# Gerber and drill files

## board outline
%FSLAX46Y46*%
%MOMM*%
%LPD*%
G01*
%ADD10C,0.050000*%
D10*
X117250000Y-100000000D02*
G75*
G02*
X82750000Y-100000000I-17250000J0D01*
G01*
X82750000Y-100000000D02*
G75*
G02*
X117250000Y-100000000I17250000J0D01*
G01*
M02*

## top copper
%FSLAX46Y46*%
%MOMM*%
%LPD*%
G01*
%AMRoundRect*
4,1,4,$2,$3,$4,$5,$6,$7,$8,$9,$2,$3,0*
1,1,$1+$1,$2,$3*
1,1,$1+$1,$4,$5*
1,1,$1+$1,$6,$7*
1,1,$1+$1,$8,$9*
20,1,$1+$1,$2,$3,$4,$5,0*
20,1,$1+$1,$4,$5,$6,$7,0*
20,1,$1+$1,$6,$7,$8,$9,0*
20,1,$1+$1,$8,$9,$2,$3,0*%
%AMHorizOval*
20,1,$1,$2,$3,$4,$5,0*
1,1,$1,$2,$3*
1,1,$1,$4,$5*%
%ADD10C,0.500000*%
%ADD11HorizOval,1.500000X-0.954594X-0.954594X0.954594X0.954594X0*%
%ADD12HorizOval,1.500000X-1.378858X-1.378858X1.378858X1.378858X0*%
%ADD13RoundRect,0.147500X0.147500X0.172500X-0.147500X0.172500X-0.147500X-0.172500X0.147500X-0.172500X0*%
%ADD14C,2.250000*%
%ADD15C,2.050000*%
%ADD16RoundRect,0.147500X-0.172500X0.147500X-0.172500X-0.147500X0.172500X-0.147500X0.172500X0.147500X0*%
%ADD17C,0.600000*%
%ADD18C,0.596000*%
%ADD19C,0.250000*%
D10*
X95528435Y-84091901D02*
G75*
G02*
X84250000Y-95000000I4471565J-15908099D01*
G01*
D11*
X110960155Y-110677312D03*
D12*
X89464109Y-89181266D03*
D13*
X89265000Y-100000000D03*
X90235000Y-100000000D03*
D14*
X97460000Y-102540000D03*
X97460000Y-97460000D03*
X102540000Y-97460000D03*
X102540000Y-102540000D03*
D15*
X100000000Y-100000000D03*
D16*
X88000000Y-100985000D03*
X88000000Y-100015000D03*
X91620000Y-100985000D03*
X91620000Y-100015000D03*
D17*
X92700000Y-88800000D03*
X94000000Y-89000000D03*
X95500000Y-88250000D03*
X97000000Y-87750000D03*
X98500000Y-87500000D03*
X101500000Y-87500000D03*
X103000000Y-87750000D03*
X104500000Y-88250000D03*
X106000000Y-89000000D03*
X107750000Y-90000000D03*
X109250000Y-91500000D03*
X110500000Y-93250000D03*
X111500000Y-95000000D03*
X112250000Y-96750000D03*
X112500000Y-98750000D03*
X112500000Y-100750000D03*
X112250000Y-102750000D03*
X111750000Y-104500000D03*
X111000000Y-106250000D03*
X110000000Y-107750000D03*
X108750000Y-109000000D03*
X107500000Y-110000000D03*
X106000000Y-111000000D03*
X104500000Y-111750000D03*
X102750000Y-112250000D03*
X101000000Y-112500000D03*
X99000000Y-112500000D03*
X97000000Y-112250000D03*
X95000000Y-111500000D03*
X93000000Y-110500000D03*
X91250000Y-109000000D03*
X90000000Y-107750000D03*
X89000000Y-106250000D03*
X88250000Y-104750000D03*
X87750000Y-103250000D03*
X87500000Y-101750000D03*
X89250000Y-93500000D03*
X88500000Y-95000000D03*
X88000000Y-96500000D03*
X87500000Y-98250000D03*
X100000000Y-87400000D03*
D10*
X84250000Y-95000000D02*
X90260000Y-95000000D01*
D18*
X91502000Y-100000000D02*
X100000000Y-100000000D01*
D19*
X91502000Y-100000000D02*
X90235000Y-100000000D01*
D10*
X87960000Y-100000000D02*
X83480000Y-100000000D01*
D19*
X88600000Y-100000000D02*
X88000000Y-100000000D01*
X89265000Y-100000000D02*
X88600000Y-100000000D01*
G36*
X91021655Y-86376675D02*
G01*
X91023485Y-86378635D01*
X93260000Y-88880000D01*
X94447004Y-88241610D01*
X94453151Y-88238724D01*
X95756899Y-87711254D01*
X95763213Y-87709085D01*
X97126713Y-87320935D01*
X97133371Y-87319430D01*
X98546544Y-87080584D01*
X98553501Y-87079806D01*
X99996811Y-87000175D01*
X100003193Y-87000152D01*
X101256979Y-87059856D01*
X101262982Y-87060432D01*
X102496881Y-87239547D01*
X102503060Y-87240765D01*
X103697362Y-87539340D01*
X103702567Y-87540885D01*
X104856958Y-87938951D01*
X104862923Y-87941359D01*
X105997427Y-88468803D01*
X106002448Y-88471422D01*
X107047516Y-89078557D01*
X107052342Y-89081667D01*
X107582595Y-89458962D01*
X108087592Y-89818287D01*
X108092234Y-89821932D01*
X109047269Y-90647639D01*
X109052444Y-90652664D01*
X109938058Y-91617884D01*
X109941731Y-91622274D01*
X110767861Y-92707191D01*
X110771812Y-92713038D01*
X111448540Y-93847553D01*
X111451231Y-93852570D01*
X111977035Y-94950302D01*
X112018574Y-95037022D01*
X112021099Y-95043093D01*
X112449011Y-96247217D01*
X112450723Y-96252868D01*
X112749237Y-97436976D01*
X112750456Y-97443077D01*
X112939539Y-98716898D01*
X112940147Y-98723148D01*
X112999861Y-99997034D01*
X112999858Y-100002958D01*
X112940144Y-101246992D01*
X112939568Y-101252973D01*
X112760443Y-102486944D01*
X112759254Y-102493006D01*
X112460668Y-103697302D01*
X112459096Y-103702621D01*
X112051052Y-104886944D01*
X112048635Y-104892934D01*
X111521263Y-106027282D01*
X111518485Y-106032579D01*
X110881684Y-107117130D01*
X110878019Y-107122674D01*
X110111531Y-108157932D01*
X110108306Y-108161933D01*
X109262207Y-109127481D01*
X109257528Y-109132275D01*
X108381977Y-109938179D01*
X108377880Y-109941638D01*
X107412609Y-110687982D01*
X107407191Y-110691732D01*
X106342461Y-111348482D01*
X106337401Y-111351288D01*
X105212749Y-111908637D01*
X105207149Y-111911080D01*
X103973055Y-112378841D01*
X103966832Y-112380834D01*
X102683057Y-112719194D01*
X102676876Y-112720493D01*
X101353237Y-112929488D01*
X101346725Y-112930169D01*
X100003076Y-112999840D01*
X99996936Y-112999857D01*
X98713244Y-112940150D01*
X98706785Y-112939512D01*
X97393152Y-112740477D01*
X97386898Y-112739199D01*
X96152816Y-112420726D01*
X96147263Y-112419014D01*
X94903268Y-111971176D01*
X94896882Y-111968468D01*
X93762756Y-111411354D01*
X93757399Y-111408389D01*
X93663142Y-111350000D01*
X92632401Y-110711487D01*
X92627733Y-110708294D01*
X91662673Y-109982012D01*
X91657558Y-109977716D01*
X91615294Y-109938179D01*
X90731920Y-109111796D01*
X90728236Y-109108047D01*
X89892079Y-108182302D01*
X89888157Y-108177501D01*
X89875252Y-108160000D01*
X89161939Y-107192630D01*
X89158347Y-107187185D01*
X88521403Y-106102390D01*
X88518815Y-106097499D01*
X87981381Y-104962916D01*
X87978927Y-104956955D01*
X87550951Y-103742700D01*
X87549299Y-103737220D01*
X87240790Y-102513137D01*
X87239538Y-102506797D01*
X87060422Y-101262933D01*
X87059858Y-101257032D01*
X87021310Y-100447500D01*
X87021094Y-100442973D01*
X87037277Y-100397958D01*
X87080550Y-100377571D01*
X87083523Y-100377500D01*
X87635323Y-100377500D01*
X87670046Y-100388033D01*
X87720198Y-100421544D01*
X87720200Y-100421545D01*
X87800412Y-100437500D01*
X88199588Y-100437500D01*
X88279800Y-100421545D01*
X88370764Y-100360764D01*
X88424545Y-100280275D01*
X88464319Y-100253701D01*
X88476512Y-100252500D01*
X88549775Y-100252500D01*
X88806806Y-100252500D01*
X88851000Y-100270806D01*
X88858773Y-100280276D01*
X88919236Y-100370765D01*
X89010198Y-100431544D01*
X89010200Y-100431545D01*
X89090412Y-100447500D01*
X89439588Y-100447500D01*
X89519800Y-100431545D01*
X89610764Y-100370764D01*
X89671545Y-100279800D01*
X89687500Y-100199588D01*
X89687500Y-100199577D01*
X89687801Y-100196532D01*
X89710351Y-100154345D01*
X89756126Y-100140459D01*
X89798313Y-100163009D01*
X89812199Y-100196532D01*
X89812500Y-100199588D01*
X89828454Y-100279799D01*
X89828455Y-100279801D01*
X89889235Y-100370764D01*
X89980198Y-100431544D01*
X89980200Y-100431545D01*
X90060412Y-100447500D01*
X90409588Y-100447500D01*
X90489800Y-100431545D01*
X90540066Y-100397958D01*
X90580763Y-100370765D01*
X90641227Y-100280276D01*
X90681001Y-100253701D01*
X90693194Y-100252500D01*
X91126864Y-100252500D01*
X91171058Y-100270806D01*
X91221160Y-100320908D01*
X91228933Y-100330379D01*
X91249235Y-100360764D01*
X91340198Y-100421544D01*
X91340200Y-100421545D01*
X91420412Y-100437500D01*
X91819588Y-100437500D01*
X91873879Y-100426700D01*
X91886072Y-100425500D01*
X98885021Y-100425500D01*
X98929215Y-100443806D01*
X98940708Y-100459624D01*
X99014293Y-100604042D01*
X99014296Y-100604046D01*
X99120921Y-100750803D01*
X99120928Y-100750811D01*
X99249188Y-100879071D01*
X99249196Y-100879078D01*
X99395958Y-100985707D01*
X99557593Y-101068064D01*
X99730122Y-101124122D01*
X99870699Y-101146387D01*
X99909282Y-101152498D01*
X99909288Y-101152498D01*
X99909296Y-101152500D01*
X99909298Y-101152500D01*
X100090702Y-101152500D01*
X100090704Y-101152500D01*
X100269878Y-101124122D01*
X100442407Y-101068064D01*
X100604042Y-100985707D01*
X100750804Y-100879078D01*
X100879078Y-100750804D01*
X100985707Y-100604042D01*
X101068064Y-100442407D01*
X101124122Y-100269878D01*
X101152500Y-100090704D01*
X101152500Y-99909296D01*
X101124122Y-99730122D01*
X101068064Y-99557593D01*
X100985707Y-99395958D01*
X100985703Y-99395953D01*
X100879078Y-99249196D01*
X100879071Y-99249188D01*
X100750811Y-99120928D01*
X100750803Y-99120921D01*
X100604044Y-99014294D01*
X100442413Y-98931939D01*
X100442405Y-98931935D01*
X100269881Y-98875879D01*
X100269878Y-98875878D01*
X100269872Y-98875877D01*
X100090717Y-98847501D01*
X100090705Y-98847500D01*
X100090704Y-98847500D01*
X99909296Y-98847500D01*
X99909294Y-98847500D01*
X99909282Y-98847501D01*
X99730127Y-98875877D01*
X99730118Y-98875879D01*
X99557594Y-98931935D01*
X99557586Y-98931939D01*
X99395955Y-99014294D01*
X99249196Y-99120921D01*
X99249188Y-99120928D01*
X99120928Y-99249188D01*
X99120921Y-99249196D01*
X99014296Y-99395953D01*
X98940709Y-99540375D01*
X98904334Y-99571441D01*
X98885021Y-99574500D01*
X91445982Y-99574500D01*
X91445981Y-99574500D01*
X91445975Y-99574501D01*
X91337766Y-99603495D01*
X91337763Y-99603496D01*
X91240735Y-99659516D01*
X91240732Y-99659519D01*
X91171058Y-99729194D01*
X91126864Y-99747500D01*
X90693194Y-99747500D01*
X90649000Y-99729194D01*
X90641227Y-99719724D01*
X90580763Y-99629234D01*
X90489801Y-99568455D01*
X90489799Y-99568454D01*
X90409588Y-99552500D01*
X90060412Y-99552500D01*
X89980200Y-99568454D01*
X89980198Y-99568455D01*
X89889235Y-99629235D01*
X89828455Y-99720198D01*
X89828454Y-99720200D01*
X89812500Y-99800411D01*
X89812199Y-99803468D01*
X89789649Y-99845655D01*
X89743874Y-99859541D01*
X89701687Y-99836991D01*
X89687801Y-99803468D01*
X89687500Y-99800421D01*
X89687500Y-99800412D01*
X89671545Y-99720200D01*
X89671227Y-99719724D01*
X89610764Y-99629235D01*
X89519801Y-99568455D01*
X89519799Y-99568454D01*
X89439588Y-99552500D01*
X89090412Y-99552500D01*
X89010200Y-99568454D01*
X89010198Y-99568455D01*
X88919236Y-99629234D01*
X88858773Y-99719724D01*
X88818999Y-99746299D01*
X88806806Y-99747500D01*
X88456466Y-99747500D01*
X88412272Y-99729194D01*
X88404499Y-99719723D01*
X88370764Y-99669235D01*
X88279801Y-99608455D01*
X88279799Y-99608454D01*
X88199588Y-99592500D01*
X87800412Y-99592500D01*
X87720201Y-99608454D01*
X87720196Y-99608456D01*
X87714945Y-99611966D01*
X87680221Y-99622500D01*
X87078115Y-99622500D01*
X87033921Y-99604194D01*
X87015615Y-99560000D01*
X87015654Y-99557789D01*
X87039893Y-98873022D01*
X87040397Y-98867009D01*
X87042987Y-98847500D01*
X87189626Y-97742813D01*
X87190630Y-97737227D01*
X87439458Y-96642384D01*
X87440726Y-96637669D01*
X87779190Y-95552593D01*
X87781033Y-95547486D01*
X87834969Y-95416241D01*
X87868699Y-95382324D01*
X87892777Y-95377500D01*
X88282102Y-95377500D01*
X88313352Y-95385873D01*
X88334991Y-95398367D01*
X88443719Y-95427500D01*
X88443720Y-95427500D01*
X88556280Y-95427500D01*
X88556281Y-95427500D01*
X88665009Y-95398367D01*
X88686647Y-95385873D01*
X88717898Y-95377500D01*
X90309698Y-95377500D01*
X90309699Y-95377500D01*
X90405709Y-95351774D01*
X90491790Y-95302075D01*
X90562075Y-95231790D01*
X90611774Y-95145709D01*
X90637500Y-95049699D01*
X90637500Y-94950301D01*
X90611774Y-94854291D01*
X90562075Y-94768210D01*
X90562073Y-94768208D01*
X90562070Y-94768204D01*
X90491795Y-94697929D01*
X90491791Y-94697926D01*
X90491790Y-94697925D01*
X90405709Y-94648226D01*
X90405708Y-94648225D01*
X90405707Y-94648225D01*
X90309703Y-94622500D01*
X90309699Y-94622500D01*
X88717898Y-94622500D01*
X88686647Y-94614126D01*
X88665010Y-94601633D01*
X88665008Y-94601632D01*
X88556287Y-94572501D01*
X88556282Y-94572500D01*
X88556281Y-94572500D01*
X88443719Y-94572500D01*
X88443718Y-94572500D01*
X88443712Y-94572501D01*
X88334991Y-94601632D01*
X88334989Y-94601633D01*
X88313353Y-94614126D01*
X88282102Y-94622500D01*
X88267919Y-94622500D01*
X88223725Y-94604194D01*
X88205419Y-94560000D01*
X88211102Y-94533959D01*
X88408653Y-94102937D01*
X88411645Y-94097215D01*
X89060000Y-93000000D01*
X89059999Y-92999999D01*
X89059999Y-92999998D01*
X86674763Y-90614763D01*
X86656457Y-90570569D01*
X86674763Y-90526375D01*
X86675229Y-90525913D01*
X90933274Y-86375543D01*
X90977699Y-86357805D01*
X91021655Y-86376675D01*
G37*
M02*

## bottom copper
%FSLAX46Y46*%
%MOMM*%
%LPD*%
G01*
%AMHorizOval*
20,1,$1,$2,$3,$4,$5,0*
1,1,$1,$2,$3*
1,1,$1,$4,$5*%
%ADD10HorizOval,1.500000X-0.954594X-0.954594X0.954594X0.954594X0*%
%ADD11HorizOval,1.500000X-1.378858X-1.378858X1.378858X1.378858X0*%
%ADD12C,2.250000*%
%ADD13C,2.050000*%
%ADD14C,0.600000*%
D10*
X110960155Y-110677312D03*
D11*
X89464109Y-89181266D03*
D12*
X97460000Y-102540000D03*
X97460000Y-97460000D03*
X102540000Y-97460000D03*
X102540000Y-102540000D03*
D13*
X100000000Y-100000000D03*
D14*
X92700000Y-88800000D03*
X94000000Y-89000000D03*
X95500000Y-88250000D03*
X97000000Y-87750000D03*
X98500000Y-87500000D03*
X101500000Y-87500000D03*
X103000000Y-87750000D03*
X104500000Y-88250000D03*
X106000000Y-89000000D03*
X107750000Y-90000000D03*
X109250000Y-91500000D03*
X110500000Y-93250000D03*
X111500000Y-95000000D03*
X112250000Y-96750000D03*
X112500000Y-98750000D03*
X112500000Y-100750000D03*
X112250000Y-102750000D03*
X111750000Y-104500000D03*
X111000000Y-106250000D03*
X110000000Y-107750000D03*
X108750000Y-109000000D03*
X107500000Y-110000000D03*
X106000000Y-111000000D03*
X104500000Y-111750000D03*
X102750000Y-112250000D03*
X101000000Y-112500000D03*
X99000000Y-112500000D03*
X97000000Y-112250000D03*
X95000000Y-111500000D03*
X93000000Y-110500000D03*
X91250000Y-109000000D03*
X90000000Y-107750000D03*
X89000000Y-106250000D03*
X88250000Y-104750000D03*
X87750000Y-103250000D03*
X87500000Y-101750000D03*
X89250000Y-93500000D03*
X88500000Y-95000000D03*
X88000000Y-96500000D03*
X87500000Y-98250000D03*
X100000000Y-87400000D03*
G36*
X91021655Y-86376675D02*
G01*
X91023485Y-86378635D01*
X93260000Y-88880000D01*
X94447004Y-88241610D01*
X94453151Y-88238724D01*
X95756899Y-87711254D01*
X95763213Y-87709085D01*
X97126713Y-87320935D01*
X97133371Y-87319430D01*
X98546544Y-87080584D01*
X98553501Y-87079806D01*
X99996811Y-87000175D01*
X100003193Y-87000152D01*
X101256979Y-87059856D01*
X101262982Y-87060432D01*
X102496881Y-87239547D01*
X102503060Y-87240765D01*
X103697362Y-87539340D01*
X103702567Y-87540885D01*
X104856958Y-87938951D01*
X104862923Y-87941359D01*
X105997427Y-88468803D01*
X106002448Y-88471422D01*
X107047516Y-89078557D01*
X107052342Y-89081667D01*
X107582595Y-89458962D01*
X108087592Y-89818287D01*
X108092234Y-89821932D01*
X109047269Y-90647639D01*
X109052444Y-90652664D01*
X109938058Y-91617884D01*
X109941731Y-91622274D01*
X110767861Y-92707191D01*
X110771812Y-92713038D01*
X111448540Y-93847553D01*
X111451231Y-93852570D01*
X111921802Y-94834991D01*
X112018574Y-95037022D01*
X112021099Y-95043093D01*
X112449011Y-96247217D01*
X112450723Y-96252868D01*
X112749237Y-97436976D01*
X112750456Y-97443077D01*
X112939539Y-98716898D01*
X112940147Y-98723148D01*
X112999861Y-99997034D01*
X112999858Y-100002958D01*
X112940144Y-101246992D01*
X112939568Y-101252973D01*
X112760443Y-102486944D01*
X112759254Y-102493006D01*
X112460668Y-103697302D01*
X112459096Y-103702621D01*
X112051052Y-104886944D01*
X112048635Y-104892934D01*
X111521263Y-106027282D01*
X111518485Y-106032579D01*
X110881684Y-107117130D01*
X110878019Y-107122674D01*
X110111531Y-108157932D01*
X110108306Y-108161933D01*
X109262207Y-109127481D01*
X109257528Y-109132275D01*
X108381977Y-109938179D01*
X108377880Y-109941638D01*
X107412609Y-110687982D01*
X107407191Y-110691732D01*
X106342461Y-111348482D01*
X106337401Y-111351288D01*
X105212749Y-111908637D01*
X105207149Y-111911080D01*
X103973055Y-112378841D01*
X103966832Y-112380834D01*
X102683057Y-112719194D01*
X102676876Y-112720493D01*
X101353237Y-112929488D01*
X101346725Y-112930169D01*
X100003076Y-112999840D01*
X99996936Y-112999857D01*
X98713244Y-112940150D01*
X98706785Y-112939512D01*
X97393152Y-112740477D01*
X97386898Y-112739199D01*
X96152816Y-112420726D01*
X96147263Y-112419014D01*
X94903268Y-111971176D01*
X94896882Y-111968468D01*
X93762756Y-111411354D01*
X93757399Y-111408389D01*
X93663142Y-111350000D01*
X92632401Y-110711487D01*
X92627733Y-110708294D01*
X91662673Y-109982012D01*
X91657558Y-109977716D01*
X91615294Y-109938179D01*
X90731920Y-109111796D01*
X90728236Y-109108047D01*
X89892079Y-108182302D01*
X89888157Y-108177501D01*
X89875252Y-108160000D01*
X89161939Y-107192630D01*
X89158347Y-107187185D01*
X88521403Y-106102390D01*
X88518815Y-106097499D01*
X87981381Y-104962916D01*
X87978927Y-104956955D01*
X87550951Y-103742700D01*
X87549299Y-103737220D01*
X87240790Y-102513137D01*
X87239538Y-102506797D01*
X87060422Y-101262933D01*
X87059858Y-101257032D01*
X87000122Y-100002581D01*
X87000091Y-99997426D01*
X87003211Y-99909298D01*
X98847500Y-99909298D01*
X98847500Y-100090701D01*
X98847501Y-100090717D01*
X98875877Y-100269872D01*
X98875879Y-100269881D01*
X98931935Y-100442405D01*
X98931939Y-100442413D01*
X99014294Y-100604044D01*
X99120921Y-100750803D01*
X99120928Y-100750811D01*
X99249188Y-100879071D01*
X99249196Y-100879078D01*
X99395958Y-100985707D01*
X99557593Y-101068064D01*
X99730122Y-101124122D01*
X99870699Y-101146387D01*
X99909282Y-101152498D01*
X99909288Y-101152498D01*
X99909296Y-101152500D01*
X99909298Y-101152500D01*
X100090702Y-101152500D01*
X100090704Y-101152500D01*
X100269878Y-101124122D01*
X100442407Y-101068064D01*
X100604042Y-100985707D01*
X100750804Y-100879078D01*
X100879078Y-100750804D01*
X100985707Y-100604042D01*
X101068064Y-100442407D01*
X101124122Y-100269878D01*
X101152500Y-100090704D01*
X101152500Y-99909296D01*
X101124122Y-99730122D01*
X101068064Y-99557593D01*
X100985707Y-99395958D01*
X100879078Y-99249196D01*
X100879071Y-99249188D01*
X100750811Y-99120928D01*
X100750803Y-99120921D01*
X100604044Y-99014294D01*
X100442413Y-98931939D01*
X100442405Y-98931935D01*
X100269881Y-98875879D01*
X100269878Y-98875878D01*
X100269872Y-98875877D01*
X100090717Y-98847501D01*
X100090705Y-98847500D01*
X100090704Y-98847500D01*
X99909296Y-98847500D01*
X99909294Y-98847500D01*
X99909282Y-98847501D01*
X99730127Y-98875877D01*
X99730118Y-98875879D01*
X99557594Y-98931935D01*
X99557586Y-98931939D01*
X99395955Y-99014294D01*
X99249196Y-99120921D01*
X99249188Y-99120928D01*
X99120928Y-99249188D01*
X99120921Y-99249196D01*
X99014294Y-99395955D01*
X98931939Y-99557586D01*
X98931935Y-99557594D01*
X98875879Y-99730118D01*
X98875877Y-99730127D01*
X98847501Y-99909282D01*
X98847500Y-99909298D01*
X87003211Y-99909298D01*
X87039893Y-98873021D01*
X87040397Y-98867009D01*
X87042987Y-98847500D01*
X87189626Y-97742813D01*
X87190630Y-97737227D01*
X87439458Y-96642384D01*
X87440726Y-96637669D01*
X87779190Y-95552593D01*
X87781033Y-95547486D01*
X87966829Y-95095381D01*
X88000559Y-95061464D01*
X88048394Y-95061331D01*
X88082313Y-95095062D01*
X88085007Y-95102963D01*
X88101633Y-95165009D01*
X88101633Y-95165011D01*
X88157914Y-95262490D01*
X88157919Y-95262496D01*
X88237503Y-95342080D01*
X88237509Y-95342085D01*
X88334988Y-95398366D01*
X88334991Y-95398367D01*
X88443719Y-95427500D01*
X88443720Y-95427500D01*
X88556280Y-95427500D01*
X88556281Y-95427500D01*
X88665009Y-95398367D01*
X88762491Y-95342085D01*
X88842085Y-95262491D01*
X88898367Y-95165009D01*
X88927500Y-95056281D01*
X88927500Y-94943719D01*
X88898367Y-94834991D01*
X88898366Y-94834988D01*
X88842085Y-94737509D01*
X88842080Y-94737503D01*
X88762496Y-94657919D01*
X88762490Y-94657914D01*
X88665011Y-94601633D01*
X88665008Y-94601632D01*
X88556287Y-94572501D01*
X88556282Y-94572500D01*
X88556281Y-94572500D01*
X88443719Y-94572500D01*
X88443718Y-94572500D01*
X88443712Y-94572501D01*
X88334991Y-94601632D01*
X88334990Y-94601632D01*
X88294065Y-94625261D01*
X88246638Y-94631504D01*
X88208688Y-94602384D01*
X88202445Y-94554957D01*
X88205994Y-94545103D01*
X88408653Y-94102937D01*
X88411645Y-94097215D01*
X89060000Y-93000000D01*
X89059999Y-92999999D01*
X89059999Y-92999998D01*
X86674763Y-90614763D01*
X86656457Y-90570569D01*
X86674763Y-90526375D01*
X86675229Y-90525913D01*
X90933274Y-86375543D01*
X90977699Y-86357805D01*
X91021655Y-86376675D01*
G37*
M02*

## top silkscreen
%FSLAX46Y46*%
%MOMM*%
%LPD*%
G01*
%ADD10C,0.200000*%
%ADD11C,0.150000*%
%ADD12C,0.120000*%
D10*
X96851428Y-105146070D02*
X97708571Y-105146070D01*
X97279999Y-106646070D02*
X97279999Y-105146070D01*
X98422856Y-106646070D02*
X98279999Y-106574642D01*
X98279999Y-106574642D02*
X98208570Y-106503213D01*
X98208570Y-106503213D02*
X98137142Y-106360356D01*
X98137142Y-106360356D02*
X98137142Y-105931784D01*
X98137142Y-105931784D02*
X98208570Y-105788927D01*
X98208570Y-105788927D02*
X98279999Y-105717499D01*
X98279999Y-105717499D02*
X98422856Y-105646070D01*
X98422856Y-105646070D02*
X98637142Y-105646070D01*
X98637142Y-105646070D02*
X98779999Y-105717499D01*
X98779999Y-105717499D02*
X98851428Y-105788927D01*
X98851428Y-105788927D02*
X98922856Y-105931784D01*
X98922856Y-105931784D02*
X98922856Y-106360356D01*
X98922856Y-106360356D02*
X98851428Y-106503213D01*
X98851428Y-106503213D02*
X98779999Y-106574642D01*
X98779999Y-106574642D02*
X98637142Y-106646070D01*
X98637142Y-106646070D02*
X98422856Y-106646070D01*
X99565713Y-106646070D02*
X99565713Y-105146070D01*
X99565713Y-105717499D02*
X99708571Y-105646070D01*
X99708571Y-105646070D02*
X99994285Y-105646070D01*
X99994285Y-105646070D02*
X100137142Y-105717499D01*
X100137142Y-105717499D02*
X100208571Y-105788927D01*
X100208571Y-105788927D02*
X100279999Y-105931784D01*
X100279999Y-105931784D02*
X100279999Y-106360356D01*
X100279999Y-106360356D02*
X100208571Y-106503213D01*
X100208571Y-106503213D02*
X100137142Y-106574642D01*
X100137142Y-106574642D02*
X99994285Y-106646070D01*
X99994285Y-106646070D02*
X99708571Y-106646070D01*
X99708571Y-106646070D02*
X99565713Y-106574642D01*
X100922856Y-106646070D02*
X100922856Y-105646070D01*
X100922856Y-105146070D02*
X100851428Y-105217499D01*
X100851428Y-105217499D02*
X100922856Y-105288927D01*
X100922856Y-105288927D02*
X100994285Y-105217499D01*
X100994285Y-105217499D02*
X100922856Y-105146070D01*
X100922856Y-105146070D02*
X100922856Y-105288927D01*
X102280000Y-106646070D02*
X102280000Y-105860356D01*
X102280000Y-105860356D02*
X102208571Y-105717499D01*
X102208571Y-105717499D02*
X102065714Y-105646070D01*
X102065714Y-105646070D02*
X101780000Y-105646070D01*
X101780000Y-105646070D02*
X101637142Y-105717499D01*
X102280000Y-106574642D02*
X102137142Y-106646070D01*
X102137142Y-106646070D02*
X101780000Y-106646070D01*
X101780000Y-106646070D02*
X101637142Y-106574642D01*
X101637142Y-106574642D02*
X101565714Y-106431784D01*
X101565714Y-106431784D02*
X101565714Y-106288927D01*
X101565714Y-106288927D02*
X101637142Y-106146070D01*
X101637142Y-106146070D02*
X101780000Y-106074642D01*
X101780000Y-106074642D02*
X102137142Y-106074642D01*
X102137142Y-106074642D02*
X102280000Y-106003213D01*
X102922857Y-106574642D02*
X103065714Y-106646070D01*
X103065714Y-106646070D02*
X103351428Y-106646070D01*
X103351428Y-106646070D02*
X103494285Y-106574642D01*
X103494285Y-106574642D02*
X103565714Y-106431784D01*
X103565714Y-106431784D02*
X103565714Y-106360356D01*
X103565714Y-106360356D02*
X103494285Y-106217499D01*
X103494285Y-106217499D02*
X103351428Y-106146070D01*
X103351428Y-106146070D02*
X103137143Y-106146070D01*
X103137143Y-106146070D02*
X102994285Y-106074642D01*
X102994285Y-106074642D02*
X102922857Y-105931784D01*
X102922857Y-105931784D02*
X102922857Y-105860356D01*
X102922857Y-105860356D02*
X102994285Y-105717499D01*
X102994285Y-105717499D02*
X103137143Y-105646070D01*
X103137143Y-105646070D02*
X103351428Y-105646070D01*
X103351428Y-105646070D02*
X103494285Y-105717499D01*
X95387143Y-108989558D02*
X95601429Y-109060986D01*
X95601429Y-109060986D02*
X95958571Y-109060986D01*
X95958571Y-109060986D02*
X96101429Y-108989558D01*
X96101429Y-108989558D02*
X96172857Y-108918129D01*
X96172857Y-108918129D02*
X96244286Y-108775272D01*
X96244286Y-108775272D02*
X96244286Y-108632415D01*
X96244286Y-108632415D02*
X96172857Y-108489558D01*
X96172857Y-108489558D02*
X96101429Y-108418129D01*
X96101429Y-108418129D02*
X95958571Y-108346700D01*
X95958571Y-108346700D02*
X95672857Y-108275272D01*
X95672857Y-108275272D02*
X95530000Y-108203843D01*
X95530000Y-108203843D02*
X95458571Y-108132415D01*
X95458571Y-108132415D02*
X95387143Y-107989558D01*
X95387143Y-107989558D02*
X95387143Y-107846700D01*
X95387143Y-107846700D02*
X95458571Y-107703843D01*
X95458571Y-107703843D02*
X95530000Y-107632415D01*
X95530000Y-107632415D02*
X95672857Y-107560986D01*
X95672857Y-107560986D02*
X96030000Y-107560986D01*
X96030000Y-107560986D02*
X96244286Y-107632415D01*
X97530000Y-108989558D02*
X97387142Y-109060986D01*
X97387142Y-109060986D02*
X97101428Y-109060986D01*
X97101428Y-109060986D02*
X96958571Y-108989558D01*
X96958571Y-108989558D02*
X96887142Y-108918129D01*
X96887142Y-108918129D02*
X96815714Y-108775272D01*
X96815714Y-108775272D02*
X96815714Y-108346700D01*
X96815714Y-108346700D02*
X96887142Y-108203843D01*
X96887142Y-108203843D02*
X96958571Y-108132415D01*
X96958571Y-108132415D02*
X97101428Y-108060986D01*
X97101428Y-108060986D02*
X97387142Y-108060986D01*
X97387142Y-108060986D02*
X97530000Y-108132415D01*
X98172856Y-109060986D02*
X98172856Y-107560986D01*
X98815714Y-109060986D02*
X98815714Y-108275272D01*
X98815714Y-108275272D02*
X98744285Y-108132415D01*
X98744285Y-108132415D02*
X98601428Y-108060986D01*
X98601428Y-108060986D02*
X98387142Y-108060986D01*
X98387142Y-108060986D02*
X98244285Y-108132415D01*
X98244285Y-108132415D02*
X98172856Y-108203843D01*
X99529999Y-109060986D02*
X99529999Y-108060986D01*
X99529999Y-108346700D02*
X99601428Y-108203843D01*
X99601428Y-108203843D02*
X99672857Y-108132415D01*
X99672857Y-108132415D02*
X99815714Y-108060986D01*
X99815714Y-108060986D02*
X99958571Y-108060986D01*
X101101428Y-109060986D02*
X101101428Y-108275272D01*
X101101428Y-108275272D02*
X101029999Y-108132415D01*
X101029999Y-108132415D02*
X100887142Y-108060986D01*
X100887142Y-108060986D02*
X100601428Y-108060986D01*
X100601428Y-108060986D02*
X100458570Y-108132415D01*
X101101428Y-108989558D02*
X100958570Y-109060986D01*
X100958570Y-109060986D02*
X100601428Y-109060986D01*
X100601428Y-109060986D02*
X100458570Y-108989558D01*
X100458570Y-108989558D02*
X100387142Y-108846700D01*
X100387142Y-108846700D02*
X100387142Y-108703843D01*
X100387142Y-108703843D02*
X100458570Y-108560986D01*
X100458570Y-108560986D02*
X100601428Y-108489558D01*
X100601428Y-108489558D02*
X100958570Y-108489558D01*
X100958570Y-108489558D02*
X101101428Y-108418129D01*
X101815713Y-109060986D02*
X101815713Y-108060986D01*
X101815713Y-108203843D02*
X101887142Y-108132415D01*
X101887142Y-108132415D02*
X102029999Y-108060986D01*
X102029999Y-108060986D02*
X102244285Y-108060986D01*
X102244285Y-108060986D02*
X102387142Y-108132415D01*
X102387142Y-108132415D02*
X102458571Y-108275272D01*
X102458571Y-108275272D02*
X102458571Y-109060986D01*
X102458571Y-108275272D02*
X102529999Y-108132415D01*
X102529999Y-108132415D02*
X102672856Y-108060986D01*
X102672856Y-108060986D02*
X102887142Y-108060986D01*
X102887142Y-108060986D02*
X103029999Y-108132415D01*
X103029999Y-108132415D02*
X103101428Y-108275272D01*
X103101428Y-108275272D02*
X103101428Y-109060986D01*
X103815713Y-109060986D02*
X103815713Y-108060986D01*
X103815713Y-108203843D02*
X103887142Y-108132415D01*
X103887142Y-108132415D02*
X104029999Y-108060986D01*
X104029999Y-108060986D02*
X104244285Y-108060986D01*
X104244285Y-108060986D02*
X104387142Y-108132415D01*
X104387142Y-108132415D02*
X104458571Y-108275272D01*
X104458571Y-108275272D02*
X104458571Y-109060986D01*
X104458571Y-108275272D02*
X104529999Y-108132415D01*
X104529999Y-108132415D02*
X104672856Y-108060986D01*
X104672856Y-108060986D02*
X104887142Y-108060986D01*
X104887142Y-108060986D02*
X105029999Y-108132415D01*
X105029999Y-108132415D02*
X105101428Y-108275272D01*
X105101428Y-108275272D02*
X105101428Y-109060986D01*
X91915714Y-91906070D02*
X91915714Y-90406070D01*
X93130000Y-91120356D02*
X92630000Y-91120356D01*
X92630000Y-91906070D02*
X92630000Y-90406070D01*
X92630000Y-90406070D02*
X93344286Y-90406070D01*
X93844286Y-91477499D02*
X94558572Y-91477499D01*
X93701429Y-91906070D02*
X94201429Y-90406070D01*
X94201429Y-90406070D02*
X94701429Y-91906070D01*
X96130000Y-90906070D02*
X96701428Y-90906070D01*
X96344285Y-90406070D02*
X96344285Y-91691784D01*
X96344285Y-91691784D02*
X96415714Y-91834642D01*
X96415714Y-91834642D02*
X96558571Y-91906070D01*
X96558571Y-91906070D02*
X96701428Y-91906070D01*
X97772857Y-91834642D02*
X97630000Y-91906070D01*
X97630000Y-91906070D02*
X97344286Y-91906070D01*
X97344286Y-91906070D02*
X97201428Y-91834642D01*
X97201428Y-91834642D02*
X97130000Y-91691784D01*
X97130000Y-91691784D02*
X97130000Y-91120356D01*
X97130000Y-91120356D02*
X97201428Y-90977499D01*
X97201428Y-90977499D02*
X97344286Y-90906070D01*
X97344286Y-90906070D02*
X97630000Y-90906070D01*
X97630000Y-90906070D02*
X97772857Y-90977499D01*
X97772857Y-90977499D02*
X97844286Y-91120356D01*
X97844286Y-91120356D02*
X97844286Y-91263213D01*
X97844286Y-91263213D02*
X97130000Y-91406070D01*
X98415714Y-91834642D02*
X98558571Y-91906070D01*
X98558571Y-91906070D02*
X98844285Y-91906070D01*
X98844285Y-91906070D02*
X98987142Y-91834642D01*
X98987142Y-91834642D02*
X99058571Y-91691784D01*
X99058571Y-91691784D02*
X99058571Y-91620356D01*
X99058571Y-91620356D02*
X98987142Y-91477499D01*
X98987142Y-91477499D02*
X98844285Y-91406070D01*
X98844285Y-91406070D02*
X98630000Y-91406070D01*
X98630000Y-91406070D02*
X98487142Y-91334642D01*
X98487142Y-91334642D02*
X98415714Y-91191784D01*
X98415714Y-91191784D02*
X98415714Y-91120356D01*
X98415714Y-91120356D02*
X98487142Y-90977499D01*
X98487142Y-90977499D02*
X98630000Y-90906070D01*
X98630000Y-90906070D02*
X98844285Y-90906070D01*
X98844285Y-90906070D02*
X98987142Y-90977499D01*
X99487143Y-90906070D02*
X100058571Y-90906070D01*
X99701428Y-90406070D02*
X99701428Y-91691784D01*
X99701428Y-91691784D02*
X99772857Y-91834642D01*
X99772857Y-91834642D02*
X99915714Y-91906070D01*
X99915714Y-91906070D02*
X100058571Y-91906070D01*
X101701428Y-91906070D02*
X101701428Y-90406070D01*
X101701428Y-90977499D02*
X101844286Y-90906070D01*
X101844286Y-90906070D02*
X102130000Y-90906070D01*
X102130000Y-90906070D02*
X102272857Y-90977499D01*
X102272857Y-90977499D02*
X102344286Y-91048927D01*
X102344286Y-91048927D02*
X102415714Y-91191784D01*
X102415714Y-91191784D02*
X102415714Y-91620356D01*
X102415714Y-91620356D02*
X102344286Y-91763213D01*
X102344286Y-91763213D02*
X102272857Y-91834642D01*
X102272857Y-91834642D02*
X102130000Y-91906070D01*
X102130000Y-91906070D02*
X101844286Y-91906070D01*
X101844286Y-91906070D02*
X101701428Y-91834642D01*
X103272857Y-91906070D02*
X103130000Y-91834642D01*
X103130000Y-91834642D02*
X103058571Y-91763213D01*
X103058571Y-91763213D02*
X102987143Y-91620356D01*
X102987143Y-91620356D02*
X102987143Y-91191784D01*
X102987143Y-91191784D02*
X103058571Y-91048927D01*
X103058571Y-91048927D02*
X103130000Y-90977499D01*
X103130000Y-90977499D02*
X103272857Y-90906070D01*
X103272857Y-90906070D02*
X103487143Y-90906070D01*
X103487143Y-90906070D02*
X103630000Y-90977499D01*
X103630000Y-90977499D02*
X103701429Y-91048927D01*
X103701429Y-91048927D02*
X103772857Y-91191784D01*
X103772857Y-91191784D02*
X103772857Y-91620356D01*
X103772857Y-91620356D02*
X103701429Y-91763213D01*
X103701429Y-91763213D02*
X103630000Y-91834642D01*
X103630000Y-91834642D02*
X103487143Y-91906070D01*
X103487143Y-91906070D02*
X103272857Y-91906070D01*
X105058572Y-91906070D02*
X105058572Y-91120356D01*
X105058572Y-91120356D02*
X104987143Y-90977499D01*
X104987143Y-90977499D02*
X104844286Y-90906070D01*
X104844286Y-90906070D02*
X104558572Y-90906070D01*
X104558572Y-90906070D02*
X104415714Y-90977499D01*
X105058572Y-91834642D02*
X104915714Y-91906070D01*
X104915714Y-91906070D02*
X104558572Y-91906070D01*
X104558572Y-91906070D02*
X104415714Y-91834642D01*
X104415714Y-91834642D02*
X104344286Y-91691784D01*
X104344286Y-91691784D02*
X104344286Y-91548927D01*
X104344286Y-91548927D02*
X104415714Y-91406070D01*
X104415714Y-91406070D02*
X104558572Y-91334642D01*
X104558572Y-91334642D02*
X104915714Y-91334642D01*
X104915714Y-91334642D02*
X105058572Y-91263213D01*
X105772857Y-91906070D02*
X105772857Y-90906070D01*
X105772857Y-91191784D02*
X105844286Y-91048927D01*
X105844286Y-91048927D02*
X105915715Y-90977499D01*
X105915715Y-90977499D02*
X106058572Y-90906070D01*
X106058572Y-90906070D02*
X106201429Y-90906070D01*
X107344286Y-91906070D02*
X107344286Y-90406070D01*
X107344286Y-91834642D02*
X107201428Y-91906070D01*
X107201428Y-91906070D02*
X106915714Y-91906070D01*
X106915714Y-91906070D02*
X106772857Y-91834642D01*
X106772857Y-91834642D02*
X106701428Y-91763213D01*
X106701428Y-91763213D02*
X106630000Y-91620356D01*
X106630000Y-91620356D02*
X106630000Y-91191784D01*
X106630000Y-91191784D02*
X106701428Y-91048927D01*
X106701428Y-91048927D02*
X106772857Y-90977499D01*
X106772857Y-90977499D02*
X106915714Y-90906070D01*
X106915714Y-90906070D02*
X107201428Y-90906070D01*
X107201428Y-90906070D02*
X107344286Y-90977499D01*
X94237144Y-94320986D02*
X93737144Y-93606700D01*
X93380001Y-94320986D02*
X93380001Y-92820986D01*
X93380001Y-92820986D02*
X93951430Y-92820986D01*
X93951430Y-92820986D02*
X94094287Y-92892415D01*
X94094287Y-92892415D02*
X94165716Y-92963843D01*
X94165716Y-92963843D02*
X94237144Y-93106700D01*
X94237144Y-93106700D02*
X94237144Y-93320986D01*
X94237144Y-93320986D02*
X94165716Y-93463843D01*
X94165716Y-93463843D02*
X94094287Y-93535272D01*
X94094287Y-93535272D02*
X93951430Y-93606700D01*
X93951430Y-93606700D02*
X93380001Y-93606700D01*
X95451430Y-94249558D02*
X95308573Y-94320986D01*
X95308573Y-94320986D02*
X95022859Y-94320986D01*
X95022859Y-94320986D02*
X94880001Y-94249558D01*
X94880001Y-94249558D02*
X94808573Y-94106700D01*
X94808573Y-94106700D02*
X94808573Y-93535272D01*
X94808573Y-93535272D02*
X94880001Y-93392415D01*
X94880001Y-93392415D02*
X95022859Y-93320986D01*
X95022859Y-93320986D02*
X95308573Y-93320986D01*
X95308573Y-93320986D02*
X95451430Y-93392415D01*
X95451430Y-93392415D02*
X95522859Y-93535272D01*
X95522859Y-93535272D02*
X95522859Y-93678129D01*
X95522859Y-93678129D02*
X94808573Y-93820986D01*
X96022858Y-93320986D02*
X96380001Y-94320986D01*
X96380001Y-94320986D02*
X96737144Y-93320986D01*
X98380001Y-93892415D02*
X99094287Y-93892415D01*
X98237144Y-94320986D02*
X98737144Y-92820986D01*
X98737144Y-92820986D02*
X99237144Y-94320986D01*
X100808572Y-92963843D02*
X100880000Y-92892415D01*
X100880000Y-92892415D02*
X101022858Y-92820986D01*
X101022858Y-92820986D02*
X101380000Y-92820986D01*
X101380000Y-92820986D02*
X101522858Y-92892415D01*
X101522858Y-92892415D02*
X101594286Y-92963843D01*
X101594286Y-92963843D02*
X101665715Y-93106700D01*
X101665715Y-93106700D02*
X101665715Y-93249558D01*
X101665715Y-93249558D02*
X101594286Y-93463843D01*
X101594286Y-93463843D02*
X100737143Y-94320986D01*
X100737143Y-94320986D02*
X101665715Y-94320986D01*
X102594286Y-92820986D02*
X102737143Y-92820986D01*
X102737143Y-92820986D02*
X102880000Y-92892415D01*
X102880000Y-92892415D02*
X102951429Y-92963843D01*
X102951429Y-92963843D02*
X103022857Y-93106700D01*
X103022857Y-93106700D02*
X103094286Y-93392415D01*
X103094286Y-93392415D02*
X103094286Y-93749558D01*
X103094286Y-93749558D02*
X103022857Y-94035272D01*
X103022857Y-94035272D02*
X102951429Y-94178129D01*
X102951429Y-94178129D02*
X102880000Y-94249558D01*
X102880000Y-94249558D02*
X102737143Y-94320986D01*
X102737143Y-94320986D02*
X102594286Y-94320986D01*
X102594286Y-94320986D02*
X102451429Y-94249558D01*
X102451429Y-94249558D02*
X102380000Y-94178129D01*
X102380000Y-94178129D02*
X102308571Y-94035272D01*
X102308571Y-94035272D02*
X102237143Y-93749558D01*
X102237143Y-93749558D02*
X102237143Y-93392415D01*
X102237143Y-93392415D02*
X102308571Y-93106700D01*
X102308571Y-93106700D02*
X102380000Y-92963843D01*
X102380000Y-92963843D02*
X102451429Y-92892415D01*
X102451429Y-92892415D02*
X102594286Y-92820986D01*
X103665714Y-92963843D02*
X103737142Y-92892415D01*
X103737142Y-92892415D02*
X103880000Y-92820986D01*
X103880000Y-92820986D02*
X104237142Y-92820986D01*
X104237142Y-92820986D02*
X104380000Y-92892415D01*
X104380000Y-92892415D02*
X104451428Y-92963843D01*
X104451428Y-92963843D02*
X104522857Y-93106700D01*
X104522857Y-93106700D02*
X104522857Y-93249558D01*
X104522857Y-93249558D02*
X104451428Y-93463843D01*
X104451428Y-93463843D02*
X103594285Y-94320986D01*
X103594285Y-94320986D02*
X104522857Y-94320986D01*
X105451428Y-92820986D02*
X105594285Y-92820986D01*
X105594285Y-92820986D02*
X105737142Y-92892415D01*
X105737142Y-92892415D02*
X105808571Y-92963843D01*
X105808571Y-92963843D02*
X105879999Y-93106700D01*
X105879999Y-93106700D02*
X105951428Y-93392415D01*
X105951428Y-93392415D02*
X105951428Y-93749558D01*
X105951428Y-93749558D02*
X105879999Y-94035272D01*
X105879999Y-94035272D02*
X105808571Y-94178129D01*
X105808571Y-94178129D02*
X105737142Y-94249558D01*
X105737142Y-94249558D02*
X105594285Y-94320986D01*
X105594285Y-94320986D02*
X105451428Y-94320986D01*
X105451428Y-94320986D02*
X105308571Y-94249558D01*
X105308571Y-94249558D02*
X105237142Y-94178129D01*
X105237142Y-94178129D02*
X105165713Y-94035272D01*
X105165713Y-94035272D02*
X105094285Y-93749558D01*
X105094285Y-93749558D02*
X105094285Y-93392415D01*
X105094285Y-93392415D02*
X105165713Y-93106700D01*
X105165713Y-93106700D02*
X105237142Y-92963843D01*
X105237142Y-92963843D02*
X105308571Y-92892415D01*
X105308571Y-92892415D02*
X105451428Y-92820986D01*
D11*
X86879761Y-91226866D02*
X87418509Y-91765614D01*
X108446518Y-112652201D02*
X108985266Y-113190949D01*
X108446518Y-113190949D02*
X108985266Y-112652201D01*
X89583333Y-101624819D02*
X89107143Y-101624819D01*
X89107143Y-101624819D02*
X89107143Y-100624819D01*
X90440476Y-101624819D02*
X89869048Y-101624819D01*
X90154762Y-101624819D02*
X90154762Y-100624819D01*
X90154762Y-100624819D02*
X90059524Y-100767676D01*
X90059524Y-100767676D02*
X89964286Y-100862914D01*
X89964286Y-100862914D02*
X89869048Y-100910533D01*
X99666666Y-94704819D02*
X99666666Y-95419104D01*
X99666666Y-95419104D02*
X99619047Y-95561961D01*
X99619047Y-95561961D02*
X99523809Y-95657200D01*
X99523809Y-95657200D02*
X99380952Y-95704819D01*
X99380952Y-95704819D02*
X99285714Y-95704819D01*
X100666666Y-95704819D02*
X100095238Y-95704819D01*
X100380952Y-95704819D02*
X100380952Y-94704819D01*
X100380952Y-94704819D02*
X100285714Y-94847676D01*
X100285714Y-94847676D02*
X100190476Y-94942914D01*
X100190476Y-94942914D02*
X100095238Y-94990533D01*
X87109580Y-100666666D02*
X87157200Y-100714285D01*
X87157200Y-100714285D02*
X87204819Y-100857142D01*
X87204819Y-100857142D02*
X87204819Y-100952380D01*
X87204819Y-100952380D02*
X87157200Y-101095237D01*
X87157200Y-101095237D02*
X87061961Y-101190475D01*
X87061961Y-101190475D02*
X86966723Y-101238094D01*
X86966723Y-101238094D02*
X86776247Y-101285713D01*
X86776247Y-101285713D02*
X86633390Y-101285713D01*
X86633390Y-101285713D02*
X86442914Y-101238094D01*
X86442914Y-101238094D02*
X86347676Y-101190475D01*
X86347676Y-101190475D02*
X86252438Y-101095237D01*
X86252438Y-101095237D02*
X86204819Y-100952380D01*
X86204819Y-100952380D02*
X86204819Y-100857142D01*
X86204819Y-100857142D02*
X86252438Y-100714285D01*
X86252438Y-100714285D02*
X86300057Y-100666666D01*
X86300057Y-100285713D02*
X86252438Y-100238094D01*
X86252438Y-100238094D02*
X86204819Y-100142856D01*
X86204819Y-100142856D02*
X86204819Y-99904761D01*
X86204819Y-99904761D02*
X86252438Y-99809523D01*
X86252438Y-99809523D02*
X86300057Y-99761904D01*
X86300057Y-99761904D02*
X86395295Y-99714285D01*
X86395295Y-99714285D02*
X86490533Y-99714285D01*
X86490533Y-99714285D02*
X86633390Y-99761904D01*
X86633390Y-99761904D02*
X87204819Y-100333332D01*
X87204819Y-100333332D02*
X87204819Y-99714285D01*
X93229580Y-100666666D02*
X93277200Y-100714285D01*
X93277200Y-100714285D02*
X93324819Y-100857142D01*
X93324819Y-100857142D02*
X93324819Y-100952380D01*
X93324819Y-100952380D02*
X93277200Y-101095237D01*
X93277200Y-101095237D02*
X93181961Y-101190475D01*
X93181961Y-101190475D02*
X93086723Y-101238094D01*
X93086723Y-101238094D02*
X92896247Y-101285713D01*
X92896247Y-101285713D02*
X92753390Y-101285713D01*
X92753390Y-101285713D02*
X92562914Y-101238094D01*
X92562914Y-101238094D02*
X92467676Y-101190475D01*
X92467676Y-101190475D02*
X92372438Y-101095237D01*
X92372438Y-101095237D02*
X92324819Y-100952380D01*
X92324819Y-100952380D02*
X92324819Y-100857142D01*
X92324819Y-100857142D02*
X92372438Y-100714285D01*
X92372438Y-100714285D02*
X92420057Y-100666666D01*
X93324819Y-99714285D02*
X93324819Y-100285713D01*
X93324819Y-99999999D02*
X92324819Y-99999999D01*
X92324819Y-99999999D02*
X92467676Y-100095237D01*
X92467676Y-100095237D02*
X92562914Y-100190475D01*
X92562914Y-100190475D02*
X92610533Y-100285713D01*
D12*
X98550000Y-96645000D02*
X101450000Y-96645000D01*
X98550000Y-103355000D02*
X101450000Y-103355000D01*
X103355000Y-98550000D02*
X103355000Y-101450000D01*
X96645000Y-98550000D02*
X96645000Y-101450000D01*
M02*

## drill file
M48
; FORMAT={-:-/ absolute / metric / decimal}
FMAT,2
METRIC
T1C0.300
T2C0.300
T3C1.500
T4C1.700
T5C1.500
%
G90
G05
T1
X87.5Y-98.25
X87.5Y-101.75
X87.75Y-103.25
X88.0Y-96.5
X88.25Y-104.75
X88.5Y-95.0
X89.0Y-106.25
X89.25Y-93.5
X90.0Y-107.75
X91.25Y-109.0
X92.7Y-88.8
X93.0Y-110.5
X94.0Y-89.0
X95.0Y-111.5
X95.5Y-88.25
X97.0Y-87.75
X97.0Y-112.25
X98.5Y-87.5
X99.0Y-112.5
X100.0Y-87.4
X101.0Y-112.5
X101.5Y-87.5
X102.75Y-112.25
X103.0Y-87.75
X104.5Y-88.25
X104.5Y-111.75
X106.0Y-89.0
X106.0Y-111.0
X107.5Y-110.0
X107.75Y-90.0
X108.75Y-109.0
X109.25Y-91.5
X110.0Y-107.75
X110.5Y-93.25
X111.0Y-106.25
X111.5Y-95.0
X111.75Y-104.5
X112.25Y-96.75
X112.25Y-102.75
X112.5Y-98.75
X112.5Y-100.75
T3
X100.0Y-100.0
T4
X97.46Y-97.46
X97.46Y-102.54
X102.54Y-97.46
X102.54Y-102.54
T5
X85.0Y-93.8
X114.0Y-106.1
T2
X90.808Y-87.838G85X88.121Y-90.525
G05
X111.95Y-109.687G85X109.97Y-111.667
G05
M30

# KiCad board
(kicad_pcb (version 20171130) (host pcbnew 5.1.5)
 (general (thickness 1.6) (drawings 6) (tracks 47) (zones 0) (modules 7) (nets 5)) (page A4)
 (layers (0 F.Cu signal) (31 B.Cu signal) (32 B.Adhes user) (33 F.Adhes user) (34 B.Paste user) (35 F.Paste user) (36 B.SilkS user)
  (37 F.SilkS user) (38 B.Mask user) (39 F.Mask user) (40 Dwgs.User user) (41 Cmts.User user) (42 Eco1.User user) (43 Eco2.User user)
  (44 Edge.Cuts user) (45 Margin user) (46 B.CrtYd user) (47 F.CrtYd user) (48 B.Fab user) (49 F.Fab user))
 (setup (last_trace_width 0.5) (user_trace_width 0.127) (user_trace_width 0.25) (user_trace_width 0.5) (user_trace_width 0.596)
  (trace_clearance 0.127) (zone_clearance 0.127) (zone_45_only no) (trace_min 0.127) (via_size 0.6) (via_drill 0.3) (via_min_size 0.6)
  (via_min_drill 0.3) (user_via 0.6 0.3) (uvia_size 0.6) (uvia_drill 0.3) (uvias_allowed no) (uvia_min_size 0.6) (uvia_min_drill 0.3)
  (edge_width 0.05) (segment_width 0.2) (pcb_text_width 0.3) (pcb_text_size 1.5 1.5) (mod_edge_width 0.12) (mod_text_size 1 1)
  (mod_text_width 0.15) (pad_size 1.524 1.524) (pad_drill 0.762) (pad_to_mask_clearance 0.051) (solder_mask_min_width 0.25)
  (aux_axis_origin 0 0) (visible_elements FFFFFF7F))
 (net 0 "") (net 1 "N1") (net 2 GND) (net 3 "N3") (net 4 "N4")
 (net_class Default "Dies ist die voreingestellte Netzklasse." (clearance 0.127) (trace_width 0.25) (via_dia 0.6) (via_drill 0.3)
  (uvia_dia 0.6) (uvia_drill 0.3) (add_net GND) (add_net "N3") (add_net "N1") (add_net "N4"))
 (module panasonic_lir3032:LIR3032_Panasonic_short (layer B.Cu) (at 100 100 315)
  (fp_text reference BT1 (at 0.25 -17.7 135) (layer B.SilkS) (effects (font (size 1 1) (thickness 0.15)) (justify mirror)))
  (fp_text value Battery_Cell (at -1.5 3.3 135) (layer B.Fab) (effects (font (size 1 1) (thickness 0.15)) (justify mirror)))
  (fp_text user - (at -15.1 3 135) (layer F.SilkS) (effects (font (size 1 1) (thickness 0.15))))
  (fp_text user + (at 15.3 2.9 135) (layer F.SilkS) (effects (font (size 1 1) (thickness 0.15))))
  (pad 1 thru_hole oval (at 15.3 -0.2 315) (size 1.5 4.2) (drill oval 0.3 3.1) (layers *.Cu *.Mask) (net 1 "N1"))
  (pad 2 thru_hole oval (at -15.1 -0.2 315) (size 1.5 5.4) (drill oval 0.3 4.1) (layers *.Cu *.Mask) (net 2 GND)))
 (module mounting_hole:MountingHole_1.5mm (layer F.Cu) (at 114 106.1)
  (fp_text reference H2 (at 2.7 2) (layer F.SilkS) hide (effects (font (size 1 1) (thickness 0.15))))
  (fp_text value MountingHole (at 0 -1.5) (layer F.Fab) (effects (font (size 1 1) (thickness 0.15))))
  (pad "" np_thru_hole oval (at 0 0) (size 1.5 1.5) (drill 1.5) (layers *.Cu *.Mask)))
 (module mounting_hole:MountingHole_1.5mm (layer F.Cu) (at 85 93.8)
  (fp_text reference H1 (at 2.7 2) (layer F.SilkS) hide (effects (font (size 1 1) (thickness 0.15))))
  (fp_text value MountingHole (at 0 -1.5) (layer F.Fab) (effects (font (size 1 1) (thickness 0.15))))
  (pad "" np_thru_hole oval (at 0 0) (size 1.5 1.5) (drill 1.5) (layers *.Cu *.Mask)))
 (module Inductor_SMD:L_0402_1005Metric (layer F.Cu) (at 89.75 100 180)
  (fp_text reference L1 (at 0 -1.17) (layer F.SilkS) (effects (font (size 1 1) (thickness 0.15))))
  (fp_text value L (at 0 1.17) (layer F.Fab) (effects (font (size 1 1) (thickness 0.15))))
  (pad 2 smd roundrect (at 0.485 0 180) (size 0.59 0.64) (layers F.Cu F.Paste F.Mask) (roundrect_rratio 0.25) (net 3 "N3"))
  (pad 1 smd roundrect (at -0.485 0 180) (size 0.59 0.64) (layers F.Cu F.Paste F.Mask) (roundrect_rratio 0.25) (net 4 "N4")))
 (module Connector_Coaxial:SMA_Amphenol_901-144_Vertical (layer F.Cu) (at 100 100)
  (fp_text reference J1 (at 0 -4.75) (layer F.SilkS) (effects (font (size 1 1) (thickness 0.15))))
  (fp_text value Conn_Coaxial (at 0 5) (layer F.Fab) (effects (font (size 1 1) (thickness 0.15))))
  (fp_line (start -1.45 -3.355) (end 1.45 -3.355) (layer F.SilkS) (width 0.12))
  (fp_line (start -1.45 3.355) (end 1.45 3.355) (layer F.SilkS) (width 0.12))
  (fp_line (start 3.355 -1.45) (end 3.355 1.45) (layer F.SilkS) (width 0.12))
  (fp_line (start -3.355 -1.45) (end -3.355 1.45) (layer F.SilkS) (width 0.12))
  (pad 2 thru_hole circle (at -2.54 2.54) (size 2.25 2.25) (drill 1.7) (layers *.Cu *.Mask) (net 2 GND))
  (pad 2 thru_hole circle (at -2.54 -2.54) (size 2.25 2.25) (drill 1.7) (layers *.Cu *.Mask) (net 2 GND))
  (pad 2 thru_hole circle (at 2.54 -2.54) (size 2.25 2.25) (drill 1.7) (layers *.Cu *.Mask) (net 2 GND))
  (pad 2 thru_hole circle (at 2.54 2.54) (size 2.25 2.25) (drill 1.7) (layers *.Cu *.Mask) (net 2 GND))
  (pad 1 thru_hole circle (at 0 0) (size 2.05 2.05) (drill 1.5) (layers *.Cu *.Mask) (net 4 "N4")))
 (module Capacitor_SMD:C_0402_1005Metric (layer F.Cu) (at 88 100.5 270)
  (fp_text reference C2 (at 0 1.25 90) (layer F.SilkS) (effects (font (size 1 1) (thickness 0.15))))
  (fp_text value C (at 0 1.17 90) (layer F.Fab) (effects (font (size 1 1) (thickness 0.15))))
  (pad 2 smd roundrect (at 0.485 0 270) (size 0.59 0.64) (layers F.Cu F.Paste F.Mask) (roundrect_rratio 0.25) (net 2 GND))
  (pad 1 smd roundrect (at -0.485 0 270) (size 0.59 0.64) (layers F.Cu F.Paste F.Mask) (roundrect_rratio 0.25) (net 3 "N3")))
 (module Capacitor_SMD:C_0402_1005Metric (layer F.Cu) (at 91.62 100.5 270)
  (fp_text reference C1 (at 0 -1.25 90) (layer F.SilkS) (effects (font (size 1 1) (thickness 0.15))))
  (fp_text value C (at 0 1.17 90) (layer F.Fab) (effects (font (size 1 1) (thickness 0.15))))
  (pad 2 smd roundrect (at 0.485 0 270) (size 0.59 0.64) (layers F.Cu F.Paste F.Mask) (roundrect_rratio 0.25) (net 2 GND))
  (pad 1 smd roundrect (at -0.485 0 270) (size 0.59 0.64) (layers F.Cu F.Paste F.Mask) (roundrect_rratio 0.25) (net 4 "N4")))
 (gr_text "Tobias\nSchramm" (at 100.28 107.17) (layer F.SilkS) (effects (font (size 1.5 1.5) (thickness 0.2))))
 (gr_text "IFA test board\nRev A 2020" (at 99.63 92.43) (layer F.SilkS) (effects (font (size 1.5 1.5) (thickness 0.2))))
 (gr_arc (start 100 100) (end 84.25 95) (angle -303.312578) (layer F.Cu) (width 0.5))
 (gr_circle (center 100 100) (end 117.25 100) (layer Edge.Cuts) (width 0.05))
 (segment (start 84.25 95) (end 90.26 95) (width 0.5) (layer F.Cu) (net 2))
 (via (at 92.7 88.8) (size 0.6) (drill 0.3) (layers F.Cu B.Cu) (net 2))
 (via (at 94 89) (size 0.6) (drill 0.3) (layers F.Cu B.Cu) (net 2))
 (via (at 95.5 88.25) (size 0.6) (drill 0.3) (layers F.Cu B.Cu) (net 2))
 (via (at 97 87.75) (size 0.6) (drill 0.3) (layers F.Cu B.Cu) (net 2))
 (via (at 98.5 87.5) (size 0.6) (drill 0.3) (layers F.Cu B.Cu) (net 2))
 (via (at 101.5 87.5) (size 0.6) (drill 0.3) (layers F.Cu B.Cu) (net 2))
 (via (at 103 87.75) (size 0.6) (drill 0.3) (layers F.Cu B.Cu) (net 2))
 (via (at 104.5 88.25) (size 0.6) (drill 0.3) (layers F.Cu B.Cu) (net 2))
 (via (at 106 89) (size 0.6) (drill 0.3) (layers F.Cu B.Cu) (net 2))
 (via (at 107.75 90) (size 0.6) (drill 0.3) (layers F.Cu B.Cu) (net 2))
 (via (at 109.25 91.5) (size 0.6) (drill 0.3) (layers F.Cu B.Cu) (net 2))
 (via (at 110.5 93.25) (size 0.6) (drill 0.3) (layers F.Cu B.Cu) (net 2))
 (via (at 111.5 95) (size 0.6) (drill 0.3) (layers F.Cu B.Cu) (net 2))
 (via (at 112.25 96.75) (size 0.6) (drill 0.3) (layers F.Cu B.Cu) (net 2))
 (via (at 112.5 98.75) (size 0.6) (drill 0.3) (layers F.Cu B.Cu) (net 2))
 (via (at 112.5 100.75) (size 0.6) (drill 0.3) (layers F.Cu B.Cu) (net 2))
 (via (at 112.25 102.75) (size 0.6) (drill 0.3) (layers F.Cu B.Cu) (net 2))
 (via (at 111.75 104.5) (size 0.6) (drill 0.3) (layers F.Cu B.Cu) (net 2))
 (via (at 111 106.25) (size 0.6) (drill 0.3) (layers F.Cu B.Cu) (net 2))
 (via (at 110 107.75) (size 0.6) (drill 0.3) (layers F.Cu B.Cu) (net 2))
 (via (at 108.75 109) (size 0.6) (drill 0.3) (layers F.Cu B.Cu) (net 2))
 (via (at 107.5 110) (size 0.6) (drill 0.3) (layers F.Cu B.Cu) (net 2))
 (via (at 106 111) (size 0.6) (drill 0.3) (layers F.Cu B.Cu) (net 2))
 (via (at 104.5 111.75) (size 0.6) (drill 0.3) (layers F.Cu B.Cu) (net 2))
 (via (at 102.75 112.25) (size 0.6) (drill 0.3) (layers F.Cu B.Cu) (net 2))
 (via (at 101 112.5) (size 0.6) (drill 0.3) (layers F.Cu B.Cu) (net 2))
 (via (at 99 112.5) (size 0.6) (drill 0.3) (layers F.Cu B.Cu) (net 2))
 (via (at 97 112.25) (size 0.6) (drill 0.3) (layers F.Cu B.Cu) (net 2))
 (via (at 95 111.5) (size 0.6) (drill 0.3) (layers F.Cu B.Cu) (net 2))
 (via (at 93 110.5) (size 0.6) (drill 0.3) (layers F.Cu B.Cu) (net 2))
 (via (at 91.25 109) (size 0.6) (drill 0.3) (layers F.Cu B.Cu) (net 2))
 (via (at 90 107.75) (size 0.6) (drill 0.3) (layers F.Cu B.Cu) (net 2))
 (via (at 89 106.25) (size 0.6) (drill 0.3) (layers F.Cu B.Cu) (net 2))
 (via (at 88.25 104.75) (size 0.6) (drill 0.3) (layers F.Cu B.Cu) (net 2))
 (via (at 87.75 103.25) (size 0.6) (drill 0.3) (layers F.Cu B.Cu) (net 2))
 (via (at 87.5 101.75) (size 0.6) (drill 0.3) (layers F.Cu B.Cu) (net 2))
 (via (at 89.25 93.5) (size 0.6) (drill 0.3) (layers F.Cu B.Cu) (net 2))
 (via (at 88.5 95) (size 0.6) (drill 0.3) (layers F.Cu B.Cu) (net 2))
 (via (at 88 96.5) (size 0.6) (drill 0.3) (layers F.Cu B.Cu) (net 2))
 (via (at 87.5 98.25) (size 0.6) (drill 0.3) (layers F.Cu B.Cu) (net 2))
 (via (at 100 87.4) (size 0.6) (drill 0.3) (layers F.Cu B.Cu) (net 2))
 (segment (start 91.502 100) (end 100 100) (width 0.596) (layer F.Cu) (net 4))
 (segment (start 91.502 100) (end 90.235 100) (width 0.25) (layer F.Cu) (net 4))
 (segment (start 87.96 100) (end 83.48 100) (width 0.5) (layer F.Cu) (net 3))
 (segment (start 88.6 100) (end 88 100) (width 0.25) (layer F.Cu) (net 3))
 (segment (start 89.265 100) (end 88.6 100) (width 0.25) (layer F.Cu) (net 3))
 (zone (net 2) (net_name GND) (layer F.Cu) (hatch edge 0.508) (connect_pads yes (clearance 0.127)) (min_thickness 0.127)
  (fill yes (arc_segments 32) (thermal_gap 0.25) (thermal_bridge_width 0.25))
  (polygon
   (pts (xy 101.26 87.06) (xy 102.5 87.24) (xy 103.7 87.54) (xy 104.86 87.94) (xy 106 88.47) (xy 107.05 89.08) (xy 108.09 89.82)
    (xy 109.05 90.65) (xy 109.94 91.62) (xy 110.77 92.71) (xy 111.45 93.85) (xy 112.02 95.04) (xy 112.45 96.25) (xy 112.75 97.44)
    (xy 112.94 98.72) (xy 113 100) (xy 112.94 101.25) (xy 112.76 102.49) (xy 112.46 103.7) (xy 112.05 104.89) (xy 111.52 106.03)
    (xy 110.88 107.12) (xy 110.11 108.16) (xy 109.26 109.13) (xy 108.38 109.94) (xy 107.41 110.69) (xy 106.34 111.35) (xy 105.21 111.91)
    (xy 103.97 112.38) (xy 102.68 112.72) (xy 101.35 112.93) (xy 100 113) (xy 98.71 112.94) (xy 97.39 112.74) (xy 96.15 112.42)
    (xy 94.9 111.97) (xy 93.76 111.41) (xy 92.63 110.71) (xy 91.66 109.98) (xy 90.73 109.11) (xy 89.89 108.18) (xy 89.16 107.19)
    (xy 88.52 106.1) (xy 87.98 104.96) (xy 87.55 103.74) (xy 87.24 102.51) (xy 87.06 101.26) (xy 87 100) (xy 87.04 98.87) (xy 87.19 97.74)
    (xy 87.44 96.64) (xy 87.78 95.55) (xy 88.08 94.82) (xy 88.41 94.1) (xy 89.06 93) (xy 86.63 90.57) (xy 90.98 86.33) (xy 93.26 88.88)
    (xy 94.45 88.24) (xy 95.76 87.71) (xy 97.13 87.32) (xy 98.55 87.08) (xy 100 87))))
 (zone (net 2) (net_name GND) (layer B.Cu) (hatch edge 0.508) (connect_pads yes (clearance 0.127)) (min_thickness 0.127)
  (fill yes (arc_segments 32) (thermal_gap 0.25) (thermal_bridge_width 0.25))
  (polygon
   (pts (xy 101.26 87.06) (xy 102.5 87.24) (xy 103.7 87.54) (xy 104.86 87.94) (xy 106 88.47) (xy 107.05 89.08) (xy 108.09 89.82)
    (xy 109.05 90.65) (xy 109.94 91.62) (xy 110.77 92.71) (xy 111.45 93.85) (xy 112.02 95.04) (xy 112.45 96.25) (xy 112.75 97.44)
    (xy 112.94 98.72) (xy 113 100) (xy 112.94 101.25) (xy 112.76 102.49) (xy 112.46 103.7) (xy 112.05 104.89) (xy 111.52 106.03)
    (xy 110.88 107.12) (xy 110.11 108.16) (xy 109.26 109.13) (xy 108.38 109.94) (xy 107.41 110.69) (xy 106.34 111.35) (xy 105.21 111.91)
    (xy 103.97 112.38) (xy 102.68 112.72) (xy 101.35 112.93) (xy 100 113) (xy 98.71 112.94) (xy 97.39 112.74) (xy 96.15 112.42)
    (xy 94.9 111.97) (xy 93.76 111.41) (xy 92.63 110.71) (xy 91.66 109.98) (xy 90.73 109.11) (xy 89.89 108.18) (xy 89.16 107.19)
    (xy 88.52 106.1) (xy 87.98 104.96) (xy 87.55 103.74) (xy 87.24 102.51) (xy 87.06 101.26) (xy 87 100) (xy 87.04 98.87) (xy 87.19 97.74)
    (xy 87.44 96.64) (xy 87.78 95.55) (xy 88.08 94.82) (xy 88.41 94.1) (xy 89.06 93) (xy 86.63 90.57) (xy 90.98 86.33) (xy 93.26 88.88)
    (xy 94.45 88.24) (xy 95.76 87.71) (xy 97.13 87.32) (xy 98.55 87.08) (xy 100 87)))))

